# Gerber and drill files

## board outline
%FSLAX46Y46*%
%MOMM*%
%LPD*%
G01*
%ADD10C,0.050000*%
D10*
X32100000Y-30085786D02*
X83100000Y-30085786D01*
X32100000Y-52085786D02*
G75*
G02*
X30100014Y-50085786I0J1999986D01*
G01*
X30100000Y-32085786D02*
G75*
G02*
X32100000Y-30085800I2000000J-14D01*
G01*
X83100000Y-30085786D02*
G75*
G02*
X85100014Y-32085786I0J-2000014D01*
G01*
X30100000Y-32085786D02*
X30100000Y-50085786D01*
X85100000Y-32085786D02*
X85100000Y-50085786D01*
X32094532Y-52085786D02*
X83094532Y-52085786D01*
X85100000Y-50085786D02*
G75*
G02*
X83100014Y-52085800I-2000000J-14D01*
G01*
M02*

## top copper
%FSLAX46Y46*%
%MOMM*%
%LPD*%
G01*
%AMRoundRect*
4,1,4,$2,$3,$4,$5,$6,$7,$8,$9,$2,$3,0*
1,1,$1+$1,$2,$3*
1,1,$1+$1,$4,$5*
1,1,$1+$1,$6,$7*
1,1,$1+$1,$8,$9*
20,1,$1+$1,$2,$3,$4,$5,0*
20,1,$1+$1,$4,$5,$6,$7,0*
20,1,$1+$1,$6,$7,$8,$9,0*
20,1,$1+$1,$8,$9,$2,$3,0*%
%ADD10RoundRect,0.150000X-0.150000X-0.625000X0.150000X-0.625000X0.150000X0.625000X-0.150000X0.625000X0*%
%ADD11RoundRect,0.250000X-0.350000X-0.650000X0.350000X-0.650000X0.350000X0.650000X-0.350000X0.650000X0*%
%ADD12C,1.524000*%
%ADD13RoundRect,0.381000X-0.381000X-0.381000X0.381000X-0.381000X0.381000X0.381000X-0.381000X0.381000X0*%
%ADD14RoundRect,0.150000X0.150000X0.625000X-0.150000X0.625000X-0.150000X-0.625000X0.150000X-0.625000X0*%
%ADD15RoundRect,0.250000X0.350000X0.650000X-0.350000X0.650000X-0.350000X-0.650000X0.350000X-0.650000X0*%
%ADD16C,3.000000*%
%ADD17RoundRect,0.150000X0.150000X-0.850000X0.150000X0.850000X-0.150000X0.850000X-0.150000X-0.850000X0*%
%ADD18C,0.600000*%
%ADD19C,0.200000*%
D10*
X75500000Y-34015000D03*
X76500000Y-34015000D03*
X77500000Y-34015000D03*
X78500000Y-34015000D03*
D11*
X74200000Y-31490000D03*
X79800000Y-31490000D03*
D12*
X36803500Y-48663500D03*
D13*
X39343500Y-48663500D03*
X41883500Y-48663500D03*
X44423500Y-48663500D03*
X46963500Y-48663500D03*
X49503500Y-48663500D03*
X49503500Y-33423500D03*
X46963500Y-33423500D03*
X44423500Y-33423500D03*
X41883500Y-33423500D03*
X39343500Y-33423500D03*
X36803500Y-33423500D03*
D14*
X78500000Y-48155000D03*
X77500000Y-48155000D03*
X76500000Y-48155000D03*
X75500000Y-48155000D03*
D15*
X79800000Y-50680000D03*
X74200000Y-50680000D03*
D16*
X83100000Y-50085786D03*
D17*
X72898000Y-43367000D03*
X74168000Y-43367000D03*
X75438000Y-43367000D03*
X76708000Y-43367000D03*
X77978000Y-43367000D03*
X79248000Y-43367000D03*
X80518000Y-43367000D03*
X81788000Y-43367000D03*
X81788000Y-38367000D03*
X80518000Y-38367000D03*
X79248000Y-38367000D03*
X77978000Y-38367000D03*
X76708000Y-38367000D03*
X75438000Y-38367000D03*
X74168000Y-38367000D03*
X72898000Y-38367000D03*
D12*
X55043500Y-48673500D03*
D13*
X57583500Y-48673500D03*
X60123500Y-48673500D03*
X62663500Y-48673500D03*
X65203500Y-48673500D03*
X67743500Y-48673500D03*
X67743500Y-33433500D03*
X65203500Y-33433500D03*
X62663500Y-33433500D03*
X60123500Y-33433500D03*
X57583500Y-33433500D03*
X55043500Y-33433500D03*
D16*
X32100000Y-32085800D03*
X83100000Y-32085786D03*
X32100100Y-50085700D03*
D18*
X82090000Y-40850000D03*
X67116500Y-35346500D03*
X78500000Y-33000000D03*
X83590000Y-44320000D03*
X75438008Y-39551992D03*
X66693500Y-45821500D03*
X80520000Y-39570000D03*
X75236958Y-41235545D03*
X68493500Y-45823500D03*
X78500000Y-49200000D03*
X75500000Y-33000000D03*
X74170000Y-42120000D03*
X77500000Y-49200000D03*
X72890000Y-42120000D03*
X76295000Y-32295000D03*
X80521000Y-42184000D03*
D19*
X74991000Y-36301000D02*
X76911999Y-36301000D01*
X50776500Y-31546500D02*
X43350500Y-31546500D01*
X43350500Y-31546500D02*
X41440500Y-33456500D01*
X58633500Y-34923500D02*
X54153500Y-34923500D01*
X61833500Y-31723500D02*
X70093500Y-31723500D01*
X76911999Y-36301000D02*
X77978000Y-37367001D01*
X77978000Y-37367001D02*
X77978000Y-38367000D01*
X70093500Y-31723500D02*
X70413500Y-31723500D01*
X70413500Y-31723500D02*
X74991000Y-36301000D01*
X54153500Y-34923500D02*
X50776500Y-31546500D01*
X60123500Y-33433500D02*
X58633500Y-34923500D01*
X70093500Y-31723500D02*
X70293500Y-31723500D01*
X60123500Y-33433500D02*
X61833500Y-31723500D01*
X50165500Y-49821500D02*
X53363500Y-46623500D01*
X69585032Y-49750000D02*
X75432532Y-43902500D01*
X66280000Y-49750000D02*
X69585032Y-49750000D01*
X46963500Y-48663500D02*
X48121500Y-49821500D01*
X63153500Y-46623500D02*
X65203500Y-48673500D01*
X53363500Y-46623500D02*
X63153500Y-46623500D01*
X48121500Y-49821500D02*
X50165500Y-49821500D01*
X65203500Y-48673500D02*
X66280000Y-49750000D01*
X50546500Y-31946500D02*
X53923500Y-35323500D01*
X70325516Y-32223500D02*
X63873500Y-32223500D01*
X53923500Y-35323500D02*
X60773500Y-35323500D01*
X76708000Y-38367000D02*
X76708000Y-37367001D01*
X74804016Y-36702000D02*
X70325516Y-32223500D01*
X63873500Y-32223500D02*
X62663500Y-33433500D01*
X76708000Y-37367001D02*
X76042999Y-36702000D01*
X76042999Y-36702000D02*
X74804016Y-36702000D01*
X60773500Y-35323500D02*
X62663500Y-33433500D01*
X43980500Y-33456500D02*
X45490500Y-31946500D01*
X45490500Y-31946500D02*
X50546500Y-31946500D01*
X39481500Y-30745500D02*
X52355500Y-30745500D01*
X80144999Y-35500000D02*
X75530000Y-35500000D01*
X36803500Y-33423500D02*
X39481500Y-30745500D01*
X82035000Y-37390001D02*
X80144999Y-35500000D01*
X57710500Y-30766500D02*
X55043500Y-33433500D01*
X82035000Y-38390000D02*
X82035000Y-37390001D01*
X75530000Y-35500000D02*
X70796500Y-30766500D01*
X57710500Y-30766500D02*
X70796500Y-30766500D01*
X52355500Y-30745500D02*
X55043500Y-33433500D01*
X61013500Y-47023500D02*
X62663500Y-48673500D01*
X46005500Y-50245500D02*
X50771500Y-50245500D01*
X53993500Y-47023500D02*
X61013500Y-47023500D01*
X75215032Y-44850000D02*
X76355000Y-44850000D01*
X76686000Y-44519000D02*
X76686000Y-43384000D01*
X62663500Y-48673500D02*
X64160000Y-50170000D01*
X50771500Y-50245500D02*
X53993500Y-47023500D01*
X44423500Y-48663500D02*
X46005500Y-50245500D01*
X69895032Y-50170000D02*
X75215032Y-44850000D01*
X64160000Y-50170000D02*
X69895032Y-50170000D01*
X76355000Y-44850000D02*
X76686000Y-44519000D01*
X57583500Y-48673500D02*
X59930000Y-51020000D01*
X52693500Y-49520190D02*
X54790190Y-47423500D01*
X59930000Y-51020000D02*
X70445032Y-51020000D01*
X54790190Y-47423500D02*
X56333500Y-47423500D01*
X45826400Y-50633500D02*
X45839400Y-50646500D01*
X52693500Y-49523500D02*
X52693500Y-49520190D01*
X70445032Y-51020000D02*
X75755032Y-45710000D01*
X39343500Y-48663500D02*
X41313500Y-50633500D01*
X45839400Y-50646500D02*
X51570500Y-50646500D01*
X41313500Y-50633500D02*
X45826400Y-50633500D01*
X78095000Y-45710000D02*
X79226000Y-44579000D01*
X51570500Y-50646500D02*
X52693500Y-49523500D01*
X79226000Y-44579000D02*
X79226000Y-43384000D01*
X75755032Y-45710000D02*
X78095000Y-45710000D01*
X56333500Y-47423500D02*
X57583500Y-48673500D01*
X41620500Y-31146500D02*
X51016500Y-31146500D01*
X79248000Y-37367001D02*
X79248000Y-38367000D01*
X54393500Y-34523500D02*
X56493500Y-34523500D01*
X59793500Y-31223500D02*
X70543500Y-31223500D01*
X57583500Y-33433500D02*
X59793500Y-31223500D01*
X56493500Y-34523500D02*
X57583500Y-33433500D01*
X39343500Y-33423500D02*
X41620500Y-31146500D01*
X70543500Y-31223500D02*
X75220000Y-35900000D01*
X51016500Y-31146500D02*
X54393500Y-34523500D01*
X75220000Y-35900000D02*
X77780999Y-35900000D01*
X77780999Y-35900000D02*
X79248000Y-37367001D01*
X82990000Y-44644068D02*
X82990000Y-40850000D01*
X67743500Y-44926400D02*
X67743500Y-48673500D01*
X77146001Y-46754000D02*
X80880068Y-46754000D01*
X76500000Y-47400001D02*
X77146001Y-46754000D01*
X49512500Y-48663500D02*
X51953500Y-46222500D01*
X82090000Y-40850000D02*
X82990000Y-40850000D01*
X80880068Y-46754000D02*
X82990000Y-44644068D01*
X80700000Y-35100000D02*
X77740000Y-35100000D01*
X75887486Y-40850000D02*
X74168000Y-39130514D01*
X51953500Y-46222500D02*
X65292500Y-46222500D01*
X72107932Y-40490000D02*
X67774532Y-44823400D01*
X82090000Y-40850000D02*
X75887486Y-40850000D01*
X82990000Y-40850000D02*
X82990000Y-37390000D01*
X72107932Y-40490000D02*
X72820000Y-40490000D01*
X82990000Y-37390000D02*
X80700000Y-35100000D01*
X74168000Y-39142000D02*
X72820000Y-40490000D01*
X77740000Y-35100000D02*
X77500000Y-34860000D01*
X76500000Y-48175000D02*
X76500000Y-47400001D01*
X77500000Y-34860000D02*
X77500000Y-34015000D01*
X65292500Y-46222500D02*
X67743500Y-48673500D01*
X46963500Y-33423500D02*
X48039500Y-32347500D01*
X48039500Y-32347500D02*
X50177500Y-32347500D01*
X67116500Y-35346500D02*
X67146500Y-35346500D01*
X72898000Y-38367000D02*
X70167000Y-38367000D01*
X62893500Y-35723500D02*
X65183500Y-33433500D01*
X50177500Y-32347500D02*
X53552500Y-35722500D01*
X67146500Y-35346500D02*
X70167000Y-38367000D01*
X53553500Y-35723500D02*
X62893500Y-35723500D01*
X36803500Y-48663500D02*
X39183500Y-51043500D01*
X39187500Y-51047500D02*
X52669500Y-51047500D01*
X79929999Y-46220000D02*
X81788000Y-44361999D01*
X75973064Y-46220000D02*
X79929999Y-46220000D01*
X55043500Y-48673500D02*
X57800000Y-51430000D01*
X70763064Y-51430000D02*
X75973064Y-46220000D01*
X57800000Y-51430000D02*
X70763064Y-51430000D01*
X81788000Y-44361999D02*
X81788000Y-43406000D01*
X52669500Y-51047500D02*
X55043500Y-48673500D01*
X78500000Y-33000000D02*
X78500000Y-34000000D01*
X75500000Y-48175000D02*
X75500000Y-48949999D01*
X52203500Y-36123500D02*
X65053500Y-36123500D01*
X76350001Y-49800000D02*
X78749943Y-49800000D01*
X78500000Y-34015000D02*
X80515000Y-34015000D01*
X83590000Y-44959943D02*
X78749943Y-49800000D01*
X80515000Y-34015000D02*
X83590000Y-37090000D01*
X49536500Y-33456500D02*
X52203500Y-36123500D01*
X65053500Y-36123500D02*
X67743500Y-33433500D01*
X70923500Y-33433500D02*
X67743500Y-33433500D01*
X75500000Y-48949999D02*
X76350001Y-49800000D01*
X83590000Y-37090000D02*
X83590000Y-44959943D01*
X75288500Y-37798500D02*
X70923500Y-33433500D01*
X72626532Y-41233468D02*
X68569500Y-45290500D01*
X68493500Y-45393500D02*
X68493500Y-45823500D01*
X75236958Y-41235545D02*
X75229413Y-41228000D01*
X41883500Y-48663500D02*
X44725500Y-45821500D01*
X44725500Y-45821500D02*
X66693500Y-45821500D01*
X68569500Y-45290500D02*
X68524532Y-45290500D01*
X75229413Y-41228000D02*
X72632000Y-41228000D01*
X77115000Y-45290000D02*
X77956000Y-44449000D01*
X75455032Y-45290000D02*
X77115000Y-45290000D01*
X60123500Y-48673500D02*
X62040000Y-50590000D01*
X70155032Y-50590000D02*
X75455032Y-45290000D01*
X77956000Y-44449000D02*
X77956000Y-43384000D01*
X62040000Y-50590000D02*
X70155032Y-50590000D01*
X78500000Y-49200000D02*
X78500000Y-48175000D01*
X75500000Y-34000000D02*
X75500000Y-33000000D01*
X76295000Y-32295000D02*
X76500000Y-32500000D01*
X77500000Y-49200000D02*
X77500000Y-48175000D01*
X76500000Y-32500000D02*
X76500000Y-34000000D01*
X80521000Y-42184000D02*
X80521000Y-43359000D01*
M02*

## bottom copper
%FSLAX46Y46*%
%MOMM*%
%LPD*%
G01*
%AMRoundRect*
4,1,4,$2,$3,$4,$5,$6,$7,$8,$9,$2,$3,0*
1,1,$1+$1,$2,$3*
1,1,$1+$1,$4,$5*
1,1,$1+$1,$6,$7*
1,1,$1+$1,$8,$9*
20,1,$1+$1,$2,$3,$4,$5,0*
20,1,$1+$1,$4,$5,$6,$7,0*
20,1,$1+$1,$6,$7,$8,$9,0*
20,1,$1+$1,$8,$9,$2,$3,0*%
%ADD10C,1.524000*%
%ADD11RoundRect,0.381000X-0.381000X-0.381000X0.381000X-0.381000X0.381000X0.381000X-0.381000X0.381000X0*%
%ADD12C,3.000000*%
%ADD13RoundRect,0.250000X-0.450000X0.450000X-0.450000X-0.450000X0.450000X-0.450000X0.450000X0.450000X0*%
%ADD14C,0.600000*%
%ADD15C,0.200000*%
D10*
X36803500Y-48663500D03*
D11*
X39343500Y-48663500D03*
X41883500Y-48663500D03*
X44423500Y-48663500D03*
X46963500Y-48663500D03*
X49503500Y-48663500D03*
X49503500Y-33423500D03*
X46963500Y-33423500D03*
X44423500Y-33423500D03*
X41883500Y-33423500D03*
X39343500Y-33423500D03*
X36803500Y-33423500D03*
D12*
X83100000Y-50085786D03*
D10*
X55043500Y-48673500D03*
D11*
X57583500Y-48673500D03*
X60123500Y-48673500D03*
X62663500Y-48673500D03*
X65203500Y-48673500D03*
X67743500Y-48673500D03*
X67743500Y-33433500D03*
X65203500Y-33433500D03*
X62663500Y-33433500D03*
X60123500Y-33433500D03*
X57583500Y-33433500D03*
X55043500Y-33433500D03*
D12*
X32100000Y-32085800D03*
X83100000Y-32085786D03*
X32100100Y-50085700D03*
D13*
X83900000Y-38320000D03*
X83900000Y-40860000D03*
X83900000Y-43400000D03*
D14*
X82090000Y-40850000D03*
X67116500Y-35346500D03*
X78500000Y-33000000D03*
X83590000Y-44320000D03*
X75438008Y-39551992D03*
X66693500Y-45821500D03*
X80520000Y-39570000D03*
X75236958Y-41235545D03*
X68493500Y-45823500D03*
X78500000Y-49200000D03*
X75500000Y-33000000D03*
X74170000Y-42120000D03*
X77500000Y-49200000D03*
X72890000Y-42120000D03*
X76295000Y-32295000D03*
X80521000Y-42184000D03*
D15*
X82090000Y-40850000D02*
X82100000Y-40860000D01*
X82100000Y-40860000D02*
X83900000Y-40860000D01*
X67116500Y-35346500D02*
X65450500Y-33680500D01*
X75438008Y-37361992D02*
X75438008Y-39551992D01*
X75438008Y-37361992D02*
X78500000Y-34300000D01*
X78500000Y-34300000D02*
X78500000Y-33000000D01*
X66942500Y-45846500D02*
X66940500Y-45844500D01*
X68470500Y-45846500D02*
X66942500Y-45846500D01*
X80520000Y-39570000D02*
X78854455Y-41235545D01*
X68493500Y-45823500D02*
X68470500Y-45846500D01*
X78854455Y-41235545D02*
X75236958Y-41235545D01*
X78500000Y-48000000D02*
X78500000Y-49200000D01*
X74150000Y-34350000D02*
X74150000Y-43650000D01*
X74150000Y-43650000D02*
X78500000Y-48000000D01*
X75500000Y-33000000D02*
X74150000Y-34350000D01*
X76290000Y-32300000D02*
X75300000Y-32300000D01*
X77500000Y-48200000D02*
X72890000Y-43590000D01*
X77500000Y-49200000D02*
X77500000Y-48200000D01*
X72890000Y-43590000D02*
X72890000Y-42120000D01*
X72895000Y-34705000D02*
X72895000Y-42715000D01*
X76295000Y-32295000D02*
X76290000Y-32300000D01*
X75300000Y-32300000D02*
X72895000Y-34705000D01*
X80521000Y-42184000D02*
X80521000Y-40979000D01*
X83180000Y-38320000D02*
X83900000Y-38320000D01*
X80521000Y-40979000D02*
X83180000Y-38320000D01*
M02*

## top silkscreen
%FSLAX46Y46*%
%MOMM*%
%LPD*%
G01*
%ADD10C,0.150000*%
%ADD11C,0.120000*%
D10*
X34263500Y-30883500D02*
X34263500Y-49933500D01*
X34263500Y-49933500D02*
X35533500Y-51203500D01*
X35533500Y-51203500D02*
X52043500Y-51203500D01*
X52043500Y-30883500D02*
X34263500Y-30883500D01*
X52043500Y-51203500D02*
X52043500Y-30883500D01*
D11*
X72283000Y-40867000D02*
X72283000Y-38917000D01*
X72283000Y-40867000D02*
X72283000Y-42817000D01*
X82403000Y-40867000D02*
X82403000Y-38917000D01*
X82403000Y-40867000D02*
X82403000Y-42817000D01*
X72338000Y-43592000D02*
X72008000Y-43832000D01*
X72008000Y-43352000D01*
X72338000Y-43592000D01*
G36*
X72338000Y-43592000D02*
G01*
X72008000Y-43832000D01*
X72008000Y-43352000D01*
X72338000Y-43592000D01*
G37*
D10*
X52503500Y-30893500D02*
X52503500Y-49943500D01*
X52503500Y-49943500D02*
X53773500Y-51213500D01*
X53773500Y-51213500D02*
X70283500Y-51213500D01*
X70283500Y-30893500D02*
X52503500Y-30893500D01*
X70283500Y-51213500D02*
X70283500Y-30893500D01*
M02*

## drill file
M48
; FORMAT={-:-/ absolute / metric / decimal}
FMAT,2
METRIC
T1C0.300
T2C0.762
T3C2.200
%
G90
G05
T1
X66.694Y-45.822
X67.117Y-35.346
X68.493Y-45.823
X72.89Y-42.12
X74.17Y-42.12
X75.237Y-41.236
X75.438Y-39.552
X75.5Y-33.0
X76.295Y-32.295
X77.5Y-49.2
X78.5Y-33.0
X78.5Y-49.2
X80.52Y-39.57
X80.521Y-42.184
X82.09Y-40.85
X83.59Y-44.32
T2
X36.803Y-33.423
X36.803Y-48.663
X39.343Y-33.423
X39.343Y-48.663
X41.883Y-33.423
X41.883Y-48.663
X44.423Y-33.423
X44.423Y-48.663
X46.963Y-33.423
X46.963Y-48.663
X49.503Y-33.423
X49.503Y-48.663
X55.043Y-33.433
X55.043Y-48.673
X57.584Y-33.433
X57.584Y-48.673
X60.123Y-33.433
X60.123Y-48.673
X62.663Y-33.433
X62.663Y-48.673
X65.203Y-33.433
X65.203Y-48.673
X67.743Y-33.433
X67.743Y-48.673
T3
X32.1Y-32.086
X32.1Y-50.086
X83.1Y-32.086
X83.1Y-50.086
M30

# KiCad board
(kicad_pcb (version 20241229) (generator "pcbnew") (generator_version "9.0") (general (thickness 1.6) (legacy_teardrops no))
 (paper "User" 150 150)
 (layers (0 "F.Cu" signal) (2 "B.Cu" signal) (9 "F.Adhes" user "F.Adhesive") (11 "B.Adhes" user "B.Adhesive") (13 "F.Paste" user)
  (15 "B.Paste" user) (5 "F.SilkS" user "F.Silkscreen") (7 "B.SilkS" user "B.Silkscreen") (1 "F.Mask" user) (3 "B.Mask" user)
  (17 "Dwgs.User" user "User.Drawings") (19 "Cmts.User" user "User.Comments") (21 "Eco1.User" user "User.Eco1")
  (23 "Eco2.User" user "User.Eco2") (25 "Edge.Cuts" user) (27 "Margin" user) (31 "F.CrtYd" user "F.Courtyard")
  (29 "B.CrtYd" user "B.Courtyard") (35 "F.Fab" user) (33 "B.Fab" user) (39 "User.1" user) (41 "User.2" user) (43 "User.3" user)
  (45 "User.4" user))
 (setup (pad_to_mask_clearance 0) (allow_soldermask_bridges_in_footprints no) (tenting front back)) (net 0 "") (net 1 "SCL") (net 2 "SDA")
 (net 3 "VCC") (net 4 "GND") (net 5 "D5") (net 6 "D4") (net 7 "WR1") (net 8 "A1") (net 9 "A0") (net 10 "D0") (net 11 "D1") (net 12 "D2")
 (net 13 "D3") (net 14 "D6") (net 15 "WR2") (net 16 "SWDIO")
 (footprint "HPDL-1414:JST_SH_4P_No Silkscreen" (layer "F.Cu") (at 77 32.69)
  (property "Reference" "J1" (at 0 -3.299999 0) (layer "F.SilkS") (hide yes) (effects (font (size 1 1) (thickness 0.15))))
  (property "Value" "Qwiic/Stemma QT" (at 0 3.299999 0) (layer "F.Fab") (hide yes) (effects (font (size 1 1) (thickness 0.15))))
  (pad "1" smd roundrect (at -1.5 1.325) (size 0.6 1.55) (layers "F.Cu" "F.Mask" "F.Paste") (roundrect_rratio 0.25) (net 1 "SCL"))
  (pad "2" smd roundrect (at -0.5 1.325) (size 0.6 1.55) (layers "F.Cu" "F.Mask" "F.Paste") (roundrect_rratio 0.25) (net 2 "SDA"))
  (pad "3" smd roundrect (at 0.5 1.325) (size 0.6 1.55) (layers "F.Cu" "F.Mask" "F.Paste") (roundrect_rratio 0.25) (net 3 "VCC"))
  (pad "4" smd roundrect (at 1.5 1.325) (size 0.6 1.55) (layers "F.Cu" "F.Mask" "F.Paste") (roundrect_rratio 0.25) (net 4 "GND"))
  (pad "MP" smd roundrect (at -2.8 -1.2) (size 1.2 1.8) (layers "F.Cu" "F.Mask" "F.Paste") (roundrect_rratio 0.208333))
  (pad "MP" smd roundrect (at 2.8 -1.2) (size 1.2 1.8) (layers "F.Cu" "F.Mask" "F.Paste") (roundrect_rratio 0.208333)))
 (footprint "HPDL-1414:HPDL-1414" (layer "F.Cu") (at 43.1535 41.0435)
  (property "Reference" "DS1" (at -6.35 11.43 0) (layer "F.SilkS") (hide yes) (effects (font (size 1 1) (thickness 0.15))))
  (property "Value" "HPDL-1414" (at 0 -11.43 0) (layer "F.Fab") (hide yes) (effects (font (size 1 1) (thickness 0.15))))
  (fp_line (start -8.89 -10.16) (end -8.89 8.89) (stroke (width 0.15) (type solid)) (layer "F.SilkS"))
  (fp_line (start -8.89 8.89) (end -7.62 10.16) (stroke (width 0.15) (type solid)) (layer "F.SilkS"))
  (fp_line (start -7.62 10.16) (end 8.89 10.16) (stroke (width 0.15) (type solid)) (layer "F.SilkS"))
  (fp_line (start 8.89 -10.16) (end -8.89 -10.16) (stroke (width 0.15) (type solid)) (layer "F.SilkS"))
  (fp_line (start 8.89 10.16) (end 8.89 -10.16) (stroke (width 0.15) (type solid)) (layer "F.SilkS"))
  (pad "1" thru_hole circle (at -6.35 7.62) (size 1.524 1.524) (drill 0.762) (layers "*.Cu" "*.Mask") (remove_unused_layers no) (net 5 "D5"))
  (pad "2" thru_hole roundrect (at -3.81 7.62) (size 1.524 1.524) (drill 0.762) (layers "*.Cu" "*.Mask") (remove_unused_layers no)
   (roundrect_rratio 0.25) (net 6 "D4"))
  (pad "3" thru_hole roundrect (at -1.27 7.62) (size 1.524 1.524) (drill 0.762) (layers "*.Cu" "*.Mask") (remove_unused_layers no)
   (roundrect_rratio 0.25) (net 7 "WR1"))
  (pad "4" thru_hole roundrect (at 1.27 7.62) (size 1.524 1.524) (drill 0.762) (layers "*.Cu" "*.Mask") (remove_unused_layers no)
   (roundrect_rratio 0.25) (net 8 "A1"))
  (pad "5" thru_hole roundrect (at 3.81 7.62) (size 1.524 1.524) (drill 0.762) (layers "*.Cu" "*.Mask") (remove_unused_layers no)
   (roundrect_rratio 0.25) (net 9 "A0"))
  (pad "6" thru_hole roundrect (at 6.35 7.62) (size 1.524 1.524) (drill 0.762) (layers "*.Cu" "*.Mask") (remove_unused_layers no)
   (roundrect_rratio 0.25) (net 3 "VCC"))
  (pad "7" thru_hole roundrect (at 6.35 -7.62) (size 1.524 1.524) (drill 0.762) (layers "*.Cu" "*.Mask") (remove_unused_layers no)
   (roundrect_rratio 0.25) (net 4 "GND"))
  (pad "8" thru_hole roundrect (at 3.81 -7.62) (size 1.524 1.524) (drill 0.762) (layers "*.Cu" "*.Mask") (remove_unused_layers no)
   (roundrect_rratio 0.25) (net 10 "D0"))
  (pad "9" thru_hole roundrect (at 1.27 -7.62) (size 1.524 1.524) (drill 0.762) (layers "*.Cu" "*.Mask") (remove_unused_layers no)
   (roundrect_rratio 0.25) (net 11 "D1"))
  (pad "10" thru_hole roundrect (at -1.27 -7.62) (size 1.524 1.524) (drill 0.762) (layers "*.Cu" "*.Mask") (remove_unused_layers no)
   (roundrect_rratio 0.25) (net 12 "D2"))
  (pad "11" thru_hole roundrect (at -3.81 -7.62) (size 1.524 1.524) (drill 0.762) (layers "*.Cu" "*.Mask") (remove_unused_layers no)
   (roundrect_rratio 0.25) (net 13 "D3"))
  (pad "12" thru_hole roundrect (at -6.35 -7.62) (size 1.524 1.524) (drill 0.762) (layers "*.Cu" "*.Mask") (remove_unused_layers no)
   (roundrect_rratio 0.25) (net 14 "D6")))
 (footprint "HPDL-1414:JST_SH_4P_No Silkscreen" (layer "F.Cu") (at 77 49.48 180)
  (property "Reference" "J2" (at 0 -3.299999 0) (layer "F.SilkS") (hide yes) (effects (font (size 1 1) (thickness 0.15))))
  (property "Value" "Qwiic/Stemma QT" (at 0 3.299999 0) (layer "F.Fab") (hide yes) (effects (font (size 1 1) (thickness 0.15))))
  (pad "1" smd roundrect (at -1.5 1.325 180) (size 0.6 1.55) (layers "F.Cu" "F.Mask" "F.Paste") (roundrect_rratio 0.25) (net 1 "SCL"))
  (pad "2" smd roundrect (at -0.5 1.325 180) (size 0.6 1.55) (layers "F.Cu" "F.Mask" "F.Paste") (roundrect_rratio 0.25) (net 2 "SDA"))
  (pad "3" smd roundrect (at 0.5 1.325 180) (size 0.6 1.55) (layers "F.Cu" "F.Mask" "F.Paste") (roundrect_rratio 0.25) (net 3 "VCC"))
  (pad "4" smd roundrect (at 1.5 1.325 180) (size 0.6 1.55) (layers "F.Cu" "F.Mask" "F.Paste") (roundrect_rratio 0.25) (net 4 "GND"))
  (pad "MP" smd roundrect (at -2.8 -1.2 180) (size 1.2 1.8) (layers "F.Cu" "F.Mask" "F.Paste") (roundrect_rratio 0.208333))
  (pad "MP" smd roundrect (at 2.8 -1.2 180) (size 1.2 1.8) (layers "F.Cu" "F.Mask" "F.Paste") (roundrect_rratio 0.208333)))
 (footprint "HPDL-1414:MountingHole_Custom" (layer "F.Cu") (at 83.1 50.085786)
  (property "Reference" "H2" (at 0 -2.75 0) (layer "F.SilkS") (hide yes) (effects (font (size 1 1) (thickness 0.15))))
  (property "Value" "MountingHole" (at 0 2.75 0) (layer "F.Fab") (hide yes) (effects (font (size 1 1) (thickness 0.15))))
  (pad "1" thru_hole circle (at 0 0) (size 3 3) (drill 2.2) (layers "*.Cu" "*.Mask") (remove_unused_layers no)))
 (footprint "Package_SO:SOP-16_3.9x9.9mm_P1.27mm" (layer "F.Cu") (at 77.343 40.867 90)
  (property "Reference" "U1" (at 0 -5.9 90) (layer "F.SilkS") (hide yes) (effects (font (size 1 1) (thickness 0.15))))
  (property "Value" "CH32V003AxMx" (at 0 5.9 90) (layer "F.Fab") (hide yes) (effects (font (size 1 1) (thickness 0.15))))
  (fp_line (start 0 -5.06) (end 1.95 -5.06) (stroke (width 0.12) (type solid)) (layer "F.SilkS"))
  (fp_line (start 0 -5.06) (end -1.95 -5.06) (stroke (width 0.12) (type solid)) (layer "F.SilkS"))
  (fp_line (start 0 5.06) (end 1.95 5.06) (stroke (width 0.12) (type solid)) (layer "F.SilkS"))
  (fp_line (start 0 5.06) (end -1.95 5.06) (stroke (width 0.12) (type solid)) (layer "F.SilkS"))
  (fp_poly (pts (xy -2.725 -5.005) (xy -2.965 -5.335) (xy -2.485 -5.335)) (stroke (width 0.12) (type solid)) (fill yes) (layer "F.SilkS"))
  (pad "1" smd roundrect (at -2.5 -4.445 90) (size 2 0.6) (layers "F.Cu" "F.Mask" "F.Paste") (roundrect_rratio 0.25) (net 2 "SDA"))
  (pad "2" smd roundrect (at -2.5 -3.175 90) (size 2 0.6) (layers "F.Cu" "F.Mask" "F.Paste") (roundrect_rratio 0.25) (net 1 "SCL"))
  (pad "3" smd roundrect (at -2.5 -1.905 90) (size 2 0.6) (layers "F.Cu" "F.Mask" "F.Paste") (roundrect_rratio 0.25) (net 9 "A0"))
  (pad "4" smd roundrect (at -2.5 -0.635 90) (size 2 0.6) (layers "F.Cu" "F.Mask" "F.Paste") (roundrect_rratio 0.25) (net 8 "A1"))
  (pad "5" smd roundrect (at -2.5 0.635 90) (size 2 0.6) (layers "F.Cu" "F.Mask" "F.Paste") (roundrect_rratio 0.25) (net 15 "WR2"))
  (pad "6" smd roundrect (at -2.5 1.905 90) (size 2 0.6) (layers "F.Cu" "F.Mask" "F.Paste") (roundrect_rratio 0.25) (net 6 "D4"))
  (pad "7" smd roundrect (at -2.5 3.175 90) (size 2 0.6) (layers "F.Cu" "F.Mask" "F.Paste") (roundrect_rratio 0.25) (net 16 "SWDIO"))
  (pad "8" smd roundrect (at -2.5 4.445 90) (size 2 0.6) (layers "F.Cu" "F.Mask" "F.Paste") (roundrect_rratio 0.25) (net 5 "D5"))
  (pad "9" smd roundrect (at 2.5 4.445 90) (size 2 0.6) (layers "F.Cu" "F.Mask" "F.Paste") (roundrect_rratio 0.25) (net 14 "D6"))
  (pad "10" smd roundrect (at 2.5 3.175 90) (size 2 0.6) (layers "F.Cu" "F.Mask" "F.Paste") (roundrect_rratio 0.25) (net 7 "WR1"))
  (pad "11" smd roundrect (at 2.5 1.905 90) (size 2 0.6) (layers "F.Cu" "F.Mask" "F.Paste") (roundrect_rratio 0.25) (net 13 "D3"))
  (pad "12" smd roundrect (at 2.5 0.635 90) (size 2 0.6) (layers "F.Cu" "F.Mask" "F.Paste") (roundrect_rratio 0.25) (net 12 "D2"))
  (pad "13" smd roundrect (at 2.5 -0.635 90) (size 2 0.6) (layers "F.Cu" "F.Mask" "F.Paste") (roundrect_rratio 0.25) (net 11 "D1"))
  (pad "14" smd roundrect (at 2.5 -1.905 90) (size 2 0.6) (layers "F.Cu" "F.Mask" "F.Paste") (roundrect_rratio 0.25) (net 4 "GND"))
  (pad "15" smd roundrect (at 2.5 -3.175 90) (size 2 0.6) (layers "F.Cu" "F.Mask" "F.Paste") (roundrect_rratio 0.25) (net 3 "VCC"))
  (pad "16" smd roundrect (at 2.5 -4.445 90) (size 2 0.6) (layers "F.Cu" "F.Mask" "F.Paste") (roundrect_rratio 0.25) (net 10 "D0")))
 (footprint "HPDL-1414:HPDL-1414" (layer "F.Cu") (at 61.3935 41.0535)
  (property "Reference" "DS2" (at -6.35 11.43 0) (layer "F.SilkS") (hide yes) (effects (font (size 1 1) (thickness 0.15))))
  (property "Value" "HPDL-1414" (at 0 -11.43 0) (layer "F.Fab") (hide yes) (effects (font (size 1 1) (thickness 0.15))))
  (fp_line (start -8.89 -10.16) (end -8.89 8.89) (stroke (width 0.15) (type solid)) (layer "F.SilkS"))
  (fp_line (start -8.89 8.89) (end -7.62 10.16) (stroke (width 0.15) (type solid)) (layer "F.SilkS"))
  (fp_line (start -7.62 10.16) (end 8.89 10.16) (stroke (width 0.15) (type solid)) (layer "F.SilkS"))
  (fp_line (start 8.89 -10.16) (end -8.89 -10.16) (stroke (width 0.15) (type solid)) (layer "F.SilkS"))
  (fp_line (start 8.89 10.16) (end 8.89 -10.16) (stroke (width 0.15) (type solid)) (layer "F.SilkS"))
  (pad "1" thru_hole circle (at -6.35 7.62) (size 1.524 1.524) (drill 0.762) (layers "*.Cu" "*.Mask") (remove_unused_layers no) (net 5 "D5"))
  (pad "2" thru_hole roundrect (at -3.81 7.62) (size 1.524 1.524) (drill 0.762) (layers "*.Cu" "*.Mask") (remove_unused_layers no)
   (roundrect_rratio 0.25) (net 6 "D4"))
  (pad "3" thru_hole roundrect (at -1.27 7.62) (size 1.524 1.524) (drill 0.762) (layers "*.Cu" "*.Mask") (remove_unused_layers no)
   (roundrect_rratio 0.25) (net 15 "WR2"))
  (pad "4" thru_hole roundrect (at 1.27 7.62) (size 1.524 1.524) (drill 0.762) (layers "*.Cu" "*.Mask") (remove_unused_layers no)
   (roundrect_rratio 0.25) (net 8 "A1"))
  (pad "5" thru_hole roundrect (at 3.81 7.62) (size 1.524 1.524) (drill 0.762) (layers "*.Cu" "*.Mask") (remove_unused_layers no)
   (roundrect_rratio 0.25) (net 9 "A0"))
  (pad "6" thru_hole roundrect (at 6.35 7.62) (size 1.524 1.524) (drill 0.762) (layers "*.Cu" "*.Mask") (remove_unused_layers no)
   (roundrect_rratio 0.25) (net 3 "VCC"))
  (pad "7" thru_hole roundrect (at 6.35 -7.62) (size 1.524 1.524) (drill 0.762) (layers "*.Cu" "*.Mask") (remove_unused_layers no)
   (roundrect_rratio 0.25) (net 4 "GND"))
  (pad "8" thru_hole roundrect (at 3.81 -7.62) (size 1.524 1.524) (drill 0.762) (layers "*.Cu" "*.Mask") (remove_unused_layers no)
   (roundrect_rratio 0.25) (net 10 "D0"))
  (pad "9" thru_hole roundrect (at 1.27 -7.62) (size 1.524 1.524) (drill 0.762) (layers "*.Cu" "*.Mask") (remove_unused_layers no)
   (roundrect_rratio 0.25) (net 11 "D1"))
  (pad "10" thru_hole roundrect (at -1.27 -7.62) (size 1.524 1.524) (drill 0.762) (layers "*.Cu" "*.Mask") (remove_unused_layers no)
   (roundrect_rratio 0.25) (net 12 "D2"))
  (pad "11" thru_hole roundrect (at -3.81 -7.62) (size 1.524 1.524) (drill 0.762) (layers "*.Cu" "*.Mask") (remove_unused_layers no)
   (roundrect_rratio 0.25) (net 13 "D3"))
  (pad "12" thru_hole roundrect (at -6.35 -7.62) (size 1.524 1.524) (drill 0.762) (layers "*.Cu" "*.Mask") (remove_unused_layers no)
   (roundrect_rratio 0.25) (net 14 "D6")))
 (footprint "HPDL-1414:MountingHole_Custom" (layer "F.Cu") (at 32.1 32.0858)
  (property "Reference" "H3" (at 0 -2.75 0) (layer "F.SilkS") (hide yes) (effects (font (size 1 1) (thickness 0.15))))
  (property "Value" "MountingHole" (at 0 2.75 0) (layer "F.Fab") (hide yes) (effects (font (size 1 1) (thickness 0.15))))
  (pad "1" thru_hole circle (at 0 0) (size 3 3) (drill 2.2) (layers "*.Cu" "*.Mask") (remove_unused_layers no)))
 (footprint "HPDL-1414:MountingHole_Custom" (layer "F.Cu") (at 83.1 32.085786)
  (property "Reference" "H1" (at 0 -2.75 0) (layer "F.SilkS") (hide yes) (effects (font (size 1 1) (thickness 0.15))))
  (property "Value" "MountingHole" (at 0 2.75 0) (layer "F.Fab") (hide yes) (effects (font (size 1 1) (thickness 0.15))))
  (pad "1" thru_hole circle (at 0 0) (size 3 3) (drill 2.2) (layers "*.Cu" "*.Mask") (remove_unused_layers no)))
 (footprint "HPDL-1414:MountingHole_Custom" (layer "F.Cu") (at 32.1001 50.0857)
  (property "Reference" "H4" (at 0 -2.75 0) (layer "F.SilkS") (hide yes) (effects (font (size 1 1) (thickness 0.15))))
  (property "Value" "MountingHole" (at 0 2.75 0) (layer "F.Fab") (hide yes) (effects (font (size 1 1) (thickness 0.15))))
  (pad "1" thru_hole circle (at 0 0) (size 3 3) (drill 2.2) (layers "*.Cu" "*.Mask") (remove_unused_layers no)))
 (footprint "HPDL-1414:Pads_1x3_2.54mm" (layer "B.Cu") (at 83.9 38.32 -90)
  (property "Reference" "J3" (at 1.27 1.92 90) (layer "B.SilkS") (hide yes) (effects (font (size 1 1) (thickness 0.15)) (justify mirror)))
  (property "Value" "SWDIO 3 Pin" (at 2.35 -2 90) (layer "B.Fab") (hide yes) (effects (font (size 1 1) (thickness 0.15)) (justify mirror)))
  (pad "1" smd roundrect (at 0 0 270) (size 1.4 1.4) (layers "B.Cu" "B.Mask") (roundrect_rratio 0.1785714286) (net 16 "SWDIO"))
  (pad "2" smd roundrect (at 2.54 0 270) (size 1.4 1.4) (layers "B.Cu" "B.Mask") (roundrect_rratio 0.1785714286) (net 3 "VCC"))
  (pad "3" smd roundrect (at 5.08 0 270) (size 1.4 1.4) (layers "B.Cu" "B.Mask") (roundrect_rratio 0.1785714286) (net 4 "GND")))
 (gr_line (start 32.1 30.085786) (end 83.1 30.085786) (stroke (width 0.05) (type solid)) (layer "Edge.Cuts"))
 (gr_arc (start 32.1 52.085786) (mid 30.685786 51.5) (end 30.1 50.085786) (stroke (width 0.05) (type default)) (layer "Edge.Cuts"))
 (gr_arc (start 30.1 32.085786) (mid 30.685786 30.671572) (end 32.1 30.085786) (stroke (width 0.05) (type default)) (layer "Edge.Cuts"))
 (gr_arc (start 83.1 30.085786) (mid 84.514214 30.671572) (end 85.1 32.085786) (stroke (width 0.05) (type default)) (layer "Edge.Cuts"))
 (gr_line (start 30.1 32.085786) (end 30.1 50.085786) (stroke (width 0.05) (type default)) (layer "Edge.Cuts"))
 (gr_line (start 85.1 32.085786) (end 85.1 50.085786) (stroke (width 0.05) (type default)) (layer "Edge.Cuts"))
 (gr_line (start 32.094532 52.085786) (end 83.094532 52.085786) (stroke (width 0.05) (type default)) (layer "Edge.Cuts"))
 (gr_arc (start 85.1 50.085786) (mid 84.514223 51.500004) (end 83.100014 52.0858) (stroke (width 0.05) (type solid)) (layer "Edge.Cuts"))
 (segment (start 74.991 36.301) (end 76.911999 36.301) (width 0.2) (layer "F.Cu") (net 12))
 (segment (start 50.7765 31.5465) (end 43.3505 31.5465) (width 0.2) (layer "F.Cu") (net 12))
 (segment (start 43.3505 31.5465) (end 41.4405 33.4565) (width 0.2) (layer "F.Cu") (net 12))
 (segment (start 58.6335 34.9235) (end 54.1535 34.9235) (width 0.2) (layer "F.Cu") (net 12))
 (segment (start 61.8335 31.7235) (end 70.0935 31.7235) (width 0.2) (layer "F.Cu") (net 12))
 (segment (start 76.911999 36.301) (end 77.978 37.367001) (width 0.2) (layer "F.Cu") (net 12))
 (segment (start 77.978 37.367001) (end 77.978 38.367) (width 0.2) (layer "F.Cu") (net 12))
 (segment (start 70.0935 31.7235) (end 70.4135 31.7235) (width 0.2) (layer "F.Cu") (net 12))
 (segment (start 70.4135 31.7235) (end 74.991 36.301) (width 0.2) (layer "F.Cu") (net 12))
 (segment (start 54.1535 34.9235) (end 50.7765 31.5465) (width 0.2) (layer "F.Cu") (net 12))
 (segment (start 60.1235 33.4335) (end 58.6335 34.9235) (width 0.2) (layer "F.Cu") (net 12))
 (segment (start 70.0935 31.7235) (end 70.2935 31.7235) (width 0.2) (layer "F.Cu") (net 12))
 (segment (start 60.1235 33.4335) (end 61.8335 31.7235) (width 0.2) (layer "F.Cu") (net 12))
 (segment (start 50.1655 49.8215) (end 53.3635 46.6235) (width 0.2) (layer "F.Cu") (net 9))
 (segment (start 69.585032 49.75) (end 75.432532 43.9025) (width 0.2) (layer "F.Cu") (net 9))
 (segment (start 66.28 49.75) (end 69.585032 49.75) (width 0.2) (layer "F.Cu") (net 9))
 (segment (start 46.9635 48.6635) (end 48.1215 49.8215) (width 0.2) (layer "F.Cu") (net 9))
 (segment (start 63.1535 46.6235) (end 65.2035 48.6735) (width 0.2) (layer "F.Cu") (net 9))
 (segment (start 53.3635 46.6235) (end 63.1535 46.6235) (width 0.2) (layer "F.Cu") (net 9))
 (segment (start 48.1215 49.8215) (end 50.1655 49.8215) (width 0.2) (layer "F.Cu") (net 9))
 (segment (start 65.2035 48.6735) (end 66.28 49.75) (width 0.2) (layer "F.Cu") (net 9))
 (segment (start 50.5465 31.9465) (end 53.9235 35.3235) (width 0.2) (layer "F.Cu") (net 11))
 (segment (start 70.325516 32.2235) (end 63.8735 32.2235) (width 0.2) (layer "F.Cu") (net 11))
 (segment (start 53.9235 35.3235) (end 60.7735 35.3235) (width 0.2) (layer "F.Cu") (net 11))
 (segment (start 76.708 38.367) (end 76.708 37.367001) (width 0.2) (layer "F.Cu") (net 11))
 (segment (start 74.804016 36.702) (end 70.325516 32.2235) (width 0.2) (layer "F.Cu") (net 11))
 (segment (start 63.8735 32.2235) (end 62.6635 33.4335) (width 0.2) (layer "F.Cu") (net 11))
 (segment (start 76.708 37.367001) (end 76.042999 36.702) (width 0.2) (layer "F.Cu") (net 11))
 (segment (start 76.042999 36.702) (end 74.804016 36.702) (width 0.2) (layer "F.Cu") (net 11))
 (segment (start 60.7735 35.3235) (end 62.6635 33.4335) (width 0.2) (layer "F.Cu") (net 11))
 (segment (start 43.9805 33.4565) (end 45.4905 31.9465) (width 0.2) (layer "F.Cu") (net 11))
 (segment (start 45.4905 31.9465) (end 50.5465 31.9465) (width 0.2) (layer "F.Cu") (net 11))
 (segment (start 39.4815 30.7455) (end 52.3555 30.7455) (width 0.2) (layer "F.Cu") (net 14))
 (segment (start 80.144999 35.5) (end 75.53 35.5) (width 0.2) (layer "F.Cu") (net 14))
 (segment (start 36.8035 33.4235) (end 39.4815 30.7455) (width 0.2) (layer "F.Cu") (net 14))
 (segment (start 82.035 37.390001) (end 80.144999 35.5) (width 0.2) (layer "F.Cu") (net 14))
 (segment (start 57.7105 30.7665) (end 55.0435 33.4335) (width 0.2) (layer "F.Cu") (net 14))
 (segment (start 82.035 38.39) (end 82.035 37.390001) (width 0.2) (layer "F.Cu") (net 14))
 (segment (start 75.53 35.5) (end 70.7965 30.7665) (width 0.2) (layer "F.Cu") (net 14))
 (segment (start 57.7105 30.7665) (end 70.7965 30.7665) (width 0.2) (layer "F.Cu") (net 14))
 (segment (start 52.3555 30.7455) (end 55.0435 33.4335) (width 0.2) (layer "F.Cu") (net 14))
 (segment (start 61.0135 47.0235) (end 62.6635 48.6735) (width 0.2) (layer "F.Cu") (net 8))
 (segment (start 46.0055 50.2455) (end 50.7715 50.2455) (width 0.2) (layer "F.Cu") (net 8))
 (segment (start 53.9935 47.0235) (end 61.0135 47.0235) (width 0.2) (layer "F.Cu") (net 8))
 (segment (start 75.215032 44.85) (end 76.355 44.85) (width 0.2) (layer "F.Cu") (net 8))
 (segment (start 76.686 44.519) (end 76.686 43.384) (width 0.2) (layer "F.Cu") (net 8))
 (segment (start 62.6635 48.6735) (end 64.16 50.17) (width 0.2) (layer "F.Cu") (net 8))
 (segment (start 50.7715 50.2455) (end 53.9935 47.0235) (width 0.2) (layer "F.Cu") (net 8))
 (segment (start 44.4235 48.6635) (end 46.0055 50.2455) (width 0.2) (layer "F.Cu") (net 8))
 (segment (start 69.895032 50.17) (end 75.215032 44.85) (width 0.2) (layer "F.Cu") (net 8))
 (segment (start 64.16 50.17) (end 69.895032 50.17) (width 0.2) (layer "F.Cu") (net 8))
 (segment (start 76.355 44.85) (end 76.686 44.519) (width 0.2) (layer "F.Cu") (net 8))
 (segment (start 57.5835 48.6735) (end 59.93 51.02) (width 0.2) (layer "F.Cu") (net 6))
 (segment (start 52.6935 49.52019) (end 54.79019 47.4235) (width 0.2) (layer "F.Cu") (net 6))
 (segment (start 59.93 51.02) (end 70.445032 51.02) (width 0.2) (layer "F.Cu") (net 6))
 (segment (start 54.79019 47.4235) (end 56.3335 47.4235) (width 0.2) (layer "F.Cu") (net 6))
 (segment (start 45.8264 50.6335) (end 45.8394 50.6465) (width 0.2) (layer "F.Cu") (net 6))
 (segment (start 52.6935 49.5235) (end 52.6935 49.52019) (width 0.2) (layer "F.Cu") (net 6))
 (segment (start 70.445032 51.02) (end 75.755032 45.71) (width 0.2) (layer "F.Cu") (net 6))
 (segment (start 39.3435 48.6635) (end 41.3135 50.6335) (width 0.2) (layer "F.Cu") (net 6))
 (segment (start 45.8394 50.6465) (end 51.5705 50.6465) (width 0.2) (layer "F.Cu") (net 6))
 (segment (start 41.3135 50.6335) (end 45.8264 50.6335) (width 0.2) (layer "F.Cu") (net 6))
 (segment (start 78.095 45.71) (end 79.226 44.579) (width 0.2) (layer "F.Cu") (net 6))
 (segment (start 51.5705 50.6465) (end 52.6935 49.5235) (width 0.2) (layer "F.Cu") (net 6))
 (segment (start 79.226 44.579) (end 79.226 43.384) (width 0.2) (layer "F.Cu") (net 6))
 (segment (start 75.755032 45.71) (end 78.095 45.71) (width 0.2) (layer "F.Cu") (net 6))
 (segment (start 56.3335 47.4235) (end 57.5835 48.6735) (width 0.2) (layer "F.Cu") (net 6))
 (segment (start 41.6205 31.1465) (end 51.0165 31.1465) (width 0.2) (layer "F.Cu") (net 13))
 (segment (start 79.248 37.367001) (end 79.248 38.367) (width 0.2) (layer "F.Cu") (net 13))
 (segment (start 54.3935 34.5235) (end 56.4935 34.5235) (width 0.2) (layer "F.Cu") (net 13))
 (segment (start 59.7935 31.2235) (end 70.5435 31.2235) (width 0.2) (layer "F.Cu") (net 13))
 (segment (start 57.5835 33.4335) (end 59.7935 31.2235) (width 0.2) (layer "F.Cu") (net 13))
 (segment (start 56.4935 34.5235) (end 57.5835 33.4335) (width 0.2) (layer "F.Cu") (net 13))
 (segment (start 39.3435 33.4235) (end 41.6205 31.1465) (width 0.2) (layer "F.Cu") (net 13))
 (segment (start 70.5435 31.2235) (end 75.22 35.9) (width 0.2) (layer "F.Cu") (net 13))
 (segment (start 51.0165 31.1465) (end 54.3935 34.5235) (width 0.2) (layer "F.Cu") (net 13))
 (segment (start 75.22 35.9) (end 77.780999 35.9) (width 0.2) (layer "F.Cu") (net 13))
 (segment (start 77.780999 35.9) (end 79.248 37.367001) (width 0.2) (layer "F.Cu") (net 13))
 (segment (start 82.99 44.644068) (end 82.99 40.85) (width 0.2) (layer "F.Cu") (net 3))
 (segment (start 67.7435 44.9264) (end 67.7435 48.6735) (width 0.2) (layer "F.Cu") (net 3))
 (segment (start 77.146001 46.754) (end 80.880068 46.754) (width 0.2) (layer "F.Cu") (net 3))
 (segment (start 76.5 47.400001) (end 77.146001 46.754) (width 0.2) (layer "F.Cu") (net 3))
 (segment (start 49.5125 48.6635) (end 51.9535 46.2225) (width 0.2) (layer "F.Cu") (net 3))
 (segment (start 82.09 40.85) (end 82.99 40.85) (width 0.2) (layer "F.Cu") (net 3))
 (segment (start 80.880068 46.754) (end 82.99 44.644068) (width 0.2) (layer "F.Cu") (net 3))
 (segment (start 80.7 35.1) (end 77.74 35.1) (width 0.2) (layer "F.Cu") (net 3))
 (segment (start 75.887486 40.85) (end 74.168 39.130514) (width 0.2) (layer "F.Cu") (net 3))
 (segment (start 51.9535 46.2225) (end 65.2925 46.2225) (width 0.2) (layer "F.Cu") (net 3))
 (segment (start 72.107932 40.49) (end 67.774532 44.8234) (width 0.2) (layer "F.Cu") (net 3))
 (segment (start 82.09 40.85) (end 75.887486 40.85) (width 0.2) (layer "F.Cu") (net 3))
 (segment (start 82.99 40.85) (end 82.99 37.39) (width 0.2) (layer "F.Cu") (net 3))
 (segment (start 72.107932 40.49) (end 72.82 40.49) (width 0.2) (layer "F.Cu") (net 3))
 (segment (start 82.99 37.39) (end 80.7 35.1) (width 0.2) (layer "F.Cu") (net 3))
 (segment (start 74.168 39.142) (end 72.82 40.49) (width 0.2) (layer "F.Cu") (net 3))
 (segment (start 77.74 35.1) (end 77.5 34.86) (width 0.2) (layer "F.Cu") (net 3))
 (segment (start 76.5 48.175) (end 76.5 47.400001) (width 0.2) (layer "F.Cu") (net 3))
 (segment (start 77.5 34.86) (end 77.5 34.015) (width 0.2) (layer "F.Cu") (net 3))
 (segment (start 65.2925 46.2225) (end 67.7435 48.6735) (width 0.2) (layer "F.Cu") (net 3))
 (via (at 82.09 40.85) (size 0.6) (drill 0.3) (layers "F.Cu" "B.Cu") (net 3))
 (segment (start 82.09 40.85) (end 82.1 40.86) (width 0.2) (layer "B.Cu") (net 3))
 (segment (start 82.1 40.86) (end 83.9 40.86) (width 0.2) (layer "B.Cu") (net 3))
 (segment (start 46.9635 33.4235) (end 48.0395 32.3475) (width 0.2) (layer "F.Cu") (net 10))
 (segment (start 48.0395 32.3475) (end 50.1775 32.3475) (width 0.2) (layer "F.Cu") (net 10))
 (segment (start 67.1165 35.3465) (end 67.1465 35.3465) (width 0.2) (layer "F.Cu") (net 10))
 (segment (start 72.898 38.367) (end 70.167 38.367) (width 0.2) (layer "F.Cu") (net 10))
 (segment (start 62.8935 35.7235) (end 65.1835 33.4335) (width 0.2) (layer "F.Cu") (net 10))
 (segment (start 50.1775 32.3475) (end 53.5525 35.7225) (width 0.2) (layer "F.Cu") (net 10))
 (segment (start 67.1465 35.3465) (end 70.167 38.367) (width 0.2) (layer "F.Cu") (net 10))
 (segment (start 53.5535 35.7235) (end 62.8935 35.7235) (width 0.2) (layer "F.Cu") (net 10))
 (via (at 67.1165 35.3465) (size 0.6) (drill 0.3) (layers "F.Cu" "B.Cu") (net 10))
 (segment (start 67.1165 35.3465) (end 65.4505 33.6805) (width 0.2) (layer "B.Cu") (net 10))
 (segment (start 36.8035 48.6635) (end 39.1835 51.0435) (width 0.2) (layer "F.Cu") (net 5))
 (segment (start 39.1875 51.0475) (end 52.6695 51.0475) (width 0.2) (layer "F.Cu") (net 5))
 (segment (start 79.929999 46.22) (end 81.788 44.361999) (width 0.2) (layer "F.Cu") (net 5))
 (segment (start 75.973064 46.22) (end 79.929999 46.22) (width 0.2) (layer "F.Cu") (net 5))
 (segment (start 55.0435 48.6735) (end 57.8 51.43) (width 0.2) (layer "F.Cu") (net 5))
 (segment (start 70.763064 51.43) (end 75.973064 46.22) (width 0.2) (layer "F.Cu") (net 5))
 (segment (start 57.8 51.43) (end 70.763064 51.43) (width 0.2) (layer "F.Cu") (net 5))
 (segment (start 81.788 44.361999) (end 81.788 43.406) (width 0.2) (layer "F.Cu") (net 5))
 (segment (start 52.6695 51.0475) (end 55.0435 48.6735) (width 0.2) (layer "F.Cu") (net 5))
 (segment (start 78.5 33) (end 78.5 34) (width 0.2) (layer "F.Cu") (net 4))
 (segment (start 75.5 48.175) (end 75.5 48.949999) (width 0.2) (layer "F.Cu") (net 4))
 (segment (start 52.2035 36.1235) (end 65.0535 36.1235) (width 0.2) (layer "F.Cu") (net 4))
 (segment (start 76.350001 49.8) (end 78.749943 49.8) (width 0.2) (layer "F.Cu") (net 4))
 (segment (start 78.5 34.015) (end 80.515 34.015) (width 0.2) (layer "F.Cu") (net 4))
 (segment (start 83.59 44.959943) (end 78.749943 49.8) (width 0.2) (layer "F.Cu") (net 4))
 (segment (start 80.515 34.015) (end 83.59 37.09) (width 0.2) (layer "F.Cu") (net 4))
 (segment (start 49.5365 33.4565) (end 52.2035 36.1235) (width 0.2) (layer "F.Cu") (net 4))
 (segment (start 65.0535 36.1235) (end 67.7435 33.4335) (width 0.2) (layer "F.Cu") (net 4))
 (segment (start 70.9235 33.4335) (end 67.7435 33.4335) (width 0.2) (layer "F.Cu") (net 4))
 (segment (start 75.5 48.949999) (end 76.350001 49.8) (width 0.2) (layer "F.Cu") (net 4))
 (segment (start 83.59 37.09) (end 83.59 44.959943) (width 0.2) (layer "F.Cu") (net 4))
 (segment (start 75.2885 37.7985) (end 70.9235 33.4335) (width 0.2) (layer "F.Cu") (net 4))
 (via (at 78.5 33) (size 0.6) (drill 0.3) (layers "F.Cu" "B.Cu") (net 4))
 (via (at 83.59 44.32) (size 0.6) (drill 0.3) (layers "F.Cu" "B.Cu") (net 4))
 (via (at 75.438008 39.551992) (size 0.6) (drill 0.3) (layers "F.Cu" "B.Cu") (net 4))
 (segment (start 75.438008 37.361992) (end 75.438008 39.551992) (width 0.2) (layer "B.Cu") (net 4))
 (segment (start 75.438008 37.361992) (end 78.5 34.3) (width 0.2) (layer "B.Cu") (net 4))
 (segment (start 78.5 34.3) (end 78.5 33) (width 0.2) (layer "B.Cu") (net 4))
 (segment (start 72.626532 41.233468) (end 68.5695 45.2905) (width 0.2) (layer "F.Cu") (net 7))
 (segment (start 68.4935 45.3935) (end 68.4935 45.8235) (width 0.2) (layer "F.Cu") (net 7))
 (segment (start 75.236958 41.235545) (end 75.229413 41.228) (width 0.2) (layer "F.Cu") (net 7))
 (segment (start 41.8835 48.6635) (end 44.7255 45.8215) (width 0.2) (layer "F.Cu") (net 7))
 (segment (start 44.7255 45.8215) (end 66.6935 45.8215) (width 0.2) (layer "F.Cu") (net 7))
 (segment (start 68.5695 45.2905) (end 68.524532 45.2905) (width 0.2) (layer "F.Cu") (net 7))
 (segment (start 75.229413 41.228) (end 72.632 41.228) (width 0.2) (layer "F.Cu") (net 7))
 (via (at 66.6935 45.8215) (size 0.6) (drill 0.3) (layers "F.Cu" "B.Cu") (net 7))
 (via (at 80.52 39.57) (size 0.6) (drill 0.3) (layers "F.Cu" "B.Cu") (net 7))
 (via (at 75.236958 41.235545) (size 0.6) (drill 0.3) (layers "F.Cu" "B.Cu") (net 7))
 (via (at 68.4935 45.8235) (size 0.6) (drill 0.3) (layers "F.Cu" "B.Cu") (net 7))
 (segment (start 66.9425 45.8465) (end 66.9405 45.8445) (width 0.2) (layer "B.Cu") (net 7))
 (segment (start 68.4705 45.8465) (end 66.9425 45.8465) (width 0.2) (layer "B.Cu") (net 7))
 (segment (start 80.52 39.57) (end 78.854455 41.235545) (width 0.2) (layer "B.Cu") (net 7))
 (segment (start 68.4935 45.8235) (end 68.4705 45.8465) (width 0.2) (layer "B.Cu") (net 7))
 (segment (start 78.854455 41.235545) (end 75.236958 41.235545) (width 0.2) (layer "B.Cu") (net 7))
 (segment (start 77.115 45.29) (end 77.956 44.449) (width 0.2) (layer "F.Cu") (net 15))
 (segment (start 75.455032 45.29) (end 77.115 45.29) (width 0.2) (layer "F.Cu") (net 15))
 (segment (start 60.1235 48.6735) (end 62.04 50.59) (width 0.2) (layer "F.Cu") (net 15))
 (segment (start 70.155032 50.59) (end 75.455032 45.29) (width 0.2) (layer "F.Cu") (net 15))
 (segment (start 77.956 44.449) (end 77.956 43.384) (width 0.2) (layer "F.Cu") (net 15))
 (segment (start 62.04 50.59) (end 70.155032 50.59) (width 0.2) (layer "F.Cu") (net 15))
 (segment (start 78.5 49.2) (end 78.5 48.175) (width 0.2) (layer "F.Cu") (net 1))
 (segment (start 75.5 34) (end 75.5 33) (width 0.2) (layer "F.Cu") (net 1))
 (via (at 78.5 49.2) (size 0.6) (drill 0.3) (layers "F.Cu" "B.Cu") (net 1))
 (via (at 75.5 33) (size 0.6) (drill 0.3) (layers "F.Cu" "B.Cu") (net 1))
 (via (at 74.17 42.12) (size 0.6) (drill 0.3) (layers "F.Cu" "B.Cu") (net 1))
 (segment (start 78.5 48) (end 78.5 49.2) (width 0.2) (layer "B.Cu") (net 1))
 (segment (start 74.15 34.35) (end 74.15 43.65) (width 0.2) (layer "B.Cu") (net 1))
 (segment (start 74.15 43.65) (end 78.5 48) (width 0.2) (layer "B.Cu") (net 1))
 (segment (start 75.5 33) (end 74.15 34.35) (width 0.2) (layer "B.Cu") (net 1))
 (segment (start 76.295 32.295) (end 76.5 32.5) (width 0.2) (layer "F.Cu") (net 2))
 (segment (start 77.5 49.2) (end 77.5 48.175) (width 0.2) (layer "F.Cu") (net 2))
 (segment (start 76.5 32.5) (end 76.5 34) (width 0.2) (layer "F.Cu") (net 2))
 (via (at 77.5 49.2) (size 0.6) (drill 0.3) (layers "F.Cu" "B.Cu") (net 2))
 (via (at 72.89 42.12) (size 0.6) (drill 0.3) (layers "F.Cu" "B.Cu") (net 2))
 (via (at 76.295 32.295) (size 0.6) (drill 0.3) (layers "F.Cu" "B.Cu") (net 2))
 (segment (start 76.29 32.3) (end 75.3 32.3) (width 0.2) (layer "B.Cu") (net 2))
 (segment (start 77.5 48.2) (end 72.89 43.59) (width 0.2) (layer "B.Cu") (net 2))
 (segment (start 77.5 49.2) (end 77.5 48.2) (width 0.2) (layer "B.Cu") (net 2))
 (segment (start 72.89 43.59) (end 72.89 42.12) (width 0.2) (layer "B.Cu") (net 2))
 (segment (start 72.895 34.705) (end 72.895 42.715) (width 0.2) (layer "B.Cu") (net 2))
 (segment (start 76.295 32.295) (end 76.29 32.3) (width 0.2) (layer "B.Cu") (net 2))
 (segment (start 75.3 32.3) (end 72.895 34.705) (width 0.2) (layer "B.Cu") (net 2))
 (segment (start 80.521 42.184) (end 80.521 43.359) (width 0.2) (layer "F.Cu") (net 16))
 (via (at 80.521 42.184) (size 0.6) (drill 0.3) (layers "F.Cu" "B.Cu") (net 16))
 (segment (start 80.521 42.184) (end 80.521 40.979) (width 0.2) (layer "B.Cu") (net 16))
 (segment (start 83.18 38.32) (end 83.9 38.32) (width 0.2) (layer "B.Cu") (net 16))
 (segment (start 80.521 40.979) (end 83.18 38.32) (width 0.2) (layer "B.Cu") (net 16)))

